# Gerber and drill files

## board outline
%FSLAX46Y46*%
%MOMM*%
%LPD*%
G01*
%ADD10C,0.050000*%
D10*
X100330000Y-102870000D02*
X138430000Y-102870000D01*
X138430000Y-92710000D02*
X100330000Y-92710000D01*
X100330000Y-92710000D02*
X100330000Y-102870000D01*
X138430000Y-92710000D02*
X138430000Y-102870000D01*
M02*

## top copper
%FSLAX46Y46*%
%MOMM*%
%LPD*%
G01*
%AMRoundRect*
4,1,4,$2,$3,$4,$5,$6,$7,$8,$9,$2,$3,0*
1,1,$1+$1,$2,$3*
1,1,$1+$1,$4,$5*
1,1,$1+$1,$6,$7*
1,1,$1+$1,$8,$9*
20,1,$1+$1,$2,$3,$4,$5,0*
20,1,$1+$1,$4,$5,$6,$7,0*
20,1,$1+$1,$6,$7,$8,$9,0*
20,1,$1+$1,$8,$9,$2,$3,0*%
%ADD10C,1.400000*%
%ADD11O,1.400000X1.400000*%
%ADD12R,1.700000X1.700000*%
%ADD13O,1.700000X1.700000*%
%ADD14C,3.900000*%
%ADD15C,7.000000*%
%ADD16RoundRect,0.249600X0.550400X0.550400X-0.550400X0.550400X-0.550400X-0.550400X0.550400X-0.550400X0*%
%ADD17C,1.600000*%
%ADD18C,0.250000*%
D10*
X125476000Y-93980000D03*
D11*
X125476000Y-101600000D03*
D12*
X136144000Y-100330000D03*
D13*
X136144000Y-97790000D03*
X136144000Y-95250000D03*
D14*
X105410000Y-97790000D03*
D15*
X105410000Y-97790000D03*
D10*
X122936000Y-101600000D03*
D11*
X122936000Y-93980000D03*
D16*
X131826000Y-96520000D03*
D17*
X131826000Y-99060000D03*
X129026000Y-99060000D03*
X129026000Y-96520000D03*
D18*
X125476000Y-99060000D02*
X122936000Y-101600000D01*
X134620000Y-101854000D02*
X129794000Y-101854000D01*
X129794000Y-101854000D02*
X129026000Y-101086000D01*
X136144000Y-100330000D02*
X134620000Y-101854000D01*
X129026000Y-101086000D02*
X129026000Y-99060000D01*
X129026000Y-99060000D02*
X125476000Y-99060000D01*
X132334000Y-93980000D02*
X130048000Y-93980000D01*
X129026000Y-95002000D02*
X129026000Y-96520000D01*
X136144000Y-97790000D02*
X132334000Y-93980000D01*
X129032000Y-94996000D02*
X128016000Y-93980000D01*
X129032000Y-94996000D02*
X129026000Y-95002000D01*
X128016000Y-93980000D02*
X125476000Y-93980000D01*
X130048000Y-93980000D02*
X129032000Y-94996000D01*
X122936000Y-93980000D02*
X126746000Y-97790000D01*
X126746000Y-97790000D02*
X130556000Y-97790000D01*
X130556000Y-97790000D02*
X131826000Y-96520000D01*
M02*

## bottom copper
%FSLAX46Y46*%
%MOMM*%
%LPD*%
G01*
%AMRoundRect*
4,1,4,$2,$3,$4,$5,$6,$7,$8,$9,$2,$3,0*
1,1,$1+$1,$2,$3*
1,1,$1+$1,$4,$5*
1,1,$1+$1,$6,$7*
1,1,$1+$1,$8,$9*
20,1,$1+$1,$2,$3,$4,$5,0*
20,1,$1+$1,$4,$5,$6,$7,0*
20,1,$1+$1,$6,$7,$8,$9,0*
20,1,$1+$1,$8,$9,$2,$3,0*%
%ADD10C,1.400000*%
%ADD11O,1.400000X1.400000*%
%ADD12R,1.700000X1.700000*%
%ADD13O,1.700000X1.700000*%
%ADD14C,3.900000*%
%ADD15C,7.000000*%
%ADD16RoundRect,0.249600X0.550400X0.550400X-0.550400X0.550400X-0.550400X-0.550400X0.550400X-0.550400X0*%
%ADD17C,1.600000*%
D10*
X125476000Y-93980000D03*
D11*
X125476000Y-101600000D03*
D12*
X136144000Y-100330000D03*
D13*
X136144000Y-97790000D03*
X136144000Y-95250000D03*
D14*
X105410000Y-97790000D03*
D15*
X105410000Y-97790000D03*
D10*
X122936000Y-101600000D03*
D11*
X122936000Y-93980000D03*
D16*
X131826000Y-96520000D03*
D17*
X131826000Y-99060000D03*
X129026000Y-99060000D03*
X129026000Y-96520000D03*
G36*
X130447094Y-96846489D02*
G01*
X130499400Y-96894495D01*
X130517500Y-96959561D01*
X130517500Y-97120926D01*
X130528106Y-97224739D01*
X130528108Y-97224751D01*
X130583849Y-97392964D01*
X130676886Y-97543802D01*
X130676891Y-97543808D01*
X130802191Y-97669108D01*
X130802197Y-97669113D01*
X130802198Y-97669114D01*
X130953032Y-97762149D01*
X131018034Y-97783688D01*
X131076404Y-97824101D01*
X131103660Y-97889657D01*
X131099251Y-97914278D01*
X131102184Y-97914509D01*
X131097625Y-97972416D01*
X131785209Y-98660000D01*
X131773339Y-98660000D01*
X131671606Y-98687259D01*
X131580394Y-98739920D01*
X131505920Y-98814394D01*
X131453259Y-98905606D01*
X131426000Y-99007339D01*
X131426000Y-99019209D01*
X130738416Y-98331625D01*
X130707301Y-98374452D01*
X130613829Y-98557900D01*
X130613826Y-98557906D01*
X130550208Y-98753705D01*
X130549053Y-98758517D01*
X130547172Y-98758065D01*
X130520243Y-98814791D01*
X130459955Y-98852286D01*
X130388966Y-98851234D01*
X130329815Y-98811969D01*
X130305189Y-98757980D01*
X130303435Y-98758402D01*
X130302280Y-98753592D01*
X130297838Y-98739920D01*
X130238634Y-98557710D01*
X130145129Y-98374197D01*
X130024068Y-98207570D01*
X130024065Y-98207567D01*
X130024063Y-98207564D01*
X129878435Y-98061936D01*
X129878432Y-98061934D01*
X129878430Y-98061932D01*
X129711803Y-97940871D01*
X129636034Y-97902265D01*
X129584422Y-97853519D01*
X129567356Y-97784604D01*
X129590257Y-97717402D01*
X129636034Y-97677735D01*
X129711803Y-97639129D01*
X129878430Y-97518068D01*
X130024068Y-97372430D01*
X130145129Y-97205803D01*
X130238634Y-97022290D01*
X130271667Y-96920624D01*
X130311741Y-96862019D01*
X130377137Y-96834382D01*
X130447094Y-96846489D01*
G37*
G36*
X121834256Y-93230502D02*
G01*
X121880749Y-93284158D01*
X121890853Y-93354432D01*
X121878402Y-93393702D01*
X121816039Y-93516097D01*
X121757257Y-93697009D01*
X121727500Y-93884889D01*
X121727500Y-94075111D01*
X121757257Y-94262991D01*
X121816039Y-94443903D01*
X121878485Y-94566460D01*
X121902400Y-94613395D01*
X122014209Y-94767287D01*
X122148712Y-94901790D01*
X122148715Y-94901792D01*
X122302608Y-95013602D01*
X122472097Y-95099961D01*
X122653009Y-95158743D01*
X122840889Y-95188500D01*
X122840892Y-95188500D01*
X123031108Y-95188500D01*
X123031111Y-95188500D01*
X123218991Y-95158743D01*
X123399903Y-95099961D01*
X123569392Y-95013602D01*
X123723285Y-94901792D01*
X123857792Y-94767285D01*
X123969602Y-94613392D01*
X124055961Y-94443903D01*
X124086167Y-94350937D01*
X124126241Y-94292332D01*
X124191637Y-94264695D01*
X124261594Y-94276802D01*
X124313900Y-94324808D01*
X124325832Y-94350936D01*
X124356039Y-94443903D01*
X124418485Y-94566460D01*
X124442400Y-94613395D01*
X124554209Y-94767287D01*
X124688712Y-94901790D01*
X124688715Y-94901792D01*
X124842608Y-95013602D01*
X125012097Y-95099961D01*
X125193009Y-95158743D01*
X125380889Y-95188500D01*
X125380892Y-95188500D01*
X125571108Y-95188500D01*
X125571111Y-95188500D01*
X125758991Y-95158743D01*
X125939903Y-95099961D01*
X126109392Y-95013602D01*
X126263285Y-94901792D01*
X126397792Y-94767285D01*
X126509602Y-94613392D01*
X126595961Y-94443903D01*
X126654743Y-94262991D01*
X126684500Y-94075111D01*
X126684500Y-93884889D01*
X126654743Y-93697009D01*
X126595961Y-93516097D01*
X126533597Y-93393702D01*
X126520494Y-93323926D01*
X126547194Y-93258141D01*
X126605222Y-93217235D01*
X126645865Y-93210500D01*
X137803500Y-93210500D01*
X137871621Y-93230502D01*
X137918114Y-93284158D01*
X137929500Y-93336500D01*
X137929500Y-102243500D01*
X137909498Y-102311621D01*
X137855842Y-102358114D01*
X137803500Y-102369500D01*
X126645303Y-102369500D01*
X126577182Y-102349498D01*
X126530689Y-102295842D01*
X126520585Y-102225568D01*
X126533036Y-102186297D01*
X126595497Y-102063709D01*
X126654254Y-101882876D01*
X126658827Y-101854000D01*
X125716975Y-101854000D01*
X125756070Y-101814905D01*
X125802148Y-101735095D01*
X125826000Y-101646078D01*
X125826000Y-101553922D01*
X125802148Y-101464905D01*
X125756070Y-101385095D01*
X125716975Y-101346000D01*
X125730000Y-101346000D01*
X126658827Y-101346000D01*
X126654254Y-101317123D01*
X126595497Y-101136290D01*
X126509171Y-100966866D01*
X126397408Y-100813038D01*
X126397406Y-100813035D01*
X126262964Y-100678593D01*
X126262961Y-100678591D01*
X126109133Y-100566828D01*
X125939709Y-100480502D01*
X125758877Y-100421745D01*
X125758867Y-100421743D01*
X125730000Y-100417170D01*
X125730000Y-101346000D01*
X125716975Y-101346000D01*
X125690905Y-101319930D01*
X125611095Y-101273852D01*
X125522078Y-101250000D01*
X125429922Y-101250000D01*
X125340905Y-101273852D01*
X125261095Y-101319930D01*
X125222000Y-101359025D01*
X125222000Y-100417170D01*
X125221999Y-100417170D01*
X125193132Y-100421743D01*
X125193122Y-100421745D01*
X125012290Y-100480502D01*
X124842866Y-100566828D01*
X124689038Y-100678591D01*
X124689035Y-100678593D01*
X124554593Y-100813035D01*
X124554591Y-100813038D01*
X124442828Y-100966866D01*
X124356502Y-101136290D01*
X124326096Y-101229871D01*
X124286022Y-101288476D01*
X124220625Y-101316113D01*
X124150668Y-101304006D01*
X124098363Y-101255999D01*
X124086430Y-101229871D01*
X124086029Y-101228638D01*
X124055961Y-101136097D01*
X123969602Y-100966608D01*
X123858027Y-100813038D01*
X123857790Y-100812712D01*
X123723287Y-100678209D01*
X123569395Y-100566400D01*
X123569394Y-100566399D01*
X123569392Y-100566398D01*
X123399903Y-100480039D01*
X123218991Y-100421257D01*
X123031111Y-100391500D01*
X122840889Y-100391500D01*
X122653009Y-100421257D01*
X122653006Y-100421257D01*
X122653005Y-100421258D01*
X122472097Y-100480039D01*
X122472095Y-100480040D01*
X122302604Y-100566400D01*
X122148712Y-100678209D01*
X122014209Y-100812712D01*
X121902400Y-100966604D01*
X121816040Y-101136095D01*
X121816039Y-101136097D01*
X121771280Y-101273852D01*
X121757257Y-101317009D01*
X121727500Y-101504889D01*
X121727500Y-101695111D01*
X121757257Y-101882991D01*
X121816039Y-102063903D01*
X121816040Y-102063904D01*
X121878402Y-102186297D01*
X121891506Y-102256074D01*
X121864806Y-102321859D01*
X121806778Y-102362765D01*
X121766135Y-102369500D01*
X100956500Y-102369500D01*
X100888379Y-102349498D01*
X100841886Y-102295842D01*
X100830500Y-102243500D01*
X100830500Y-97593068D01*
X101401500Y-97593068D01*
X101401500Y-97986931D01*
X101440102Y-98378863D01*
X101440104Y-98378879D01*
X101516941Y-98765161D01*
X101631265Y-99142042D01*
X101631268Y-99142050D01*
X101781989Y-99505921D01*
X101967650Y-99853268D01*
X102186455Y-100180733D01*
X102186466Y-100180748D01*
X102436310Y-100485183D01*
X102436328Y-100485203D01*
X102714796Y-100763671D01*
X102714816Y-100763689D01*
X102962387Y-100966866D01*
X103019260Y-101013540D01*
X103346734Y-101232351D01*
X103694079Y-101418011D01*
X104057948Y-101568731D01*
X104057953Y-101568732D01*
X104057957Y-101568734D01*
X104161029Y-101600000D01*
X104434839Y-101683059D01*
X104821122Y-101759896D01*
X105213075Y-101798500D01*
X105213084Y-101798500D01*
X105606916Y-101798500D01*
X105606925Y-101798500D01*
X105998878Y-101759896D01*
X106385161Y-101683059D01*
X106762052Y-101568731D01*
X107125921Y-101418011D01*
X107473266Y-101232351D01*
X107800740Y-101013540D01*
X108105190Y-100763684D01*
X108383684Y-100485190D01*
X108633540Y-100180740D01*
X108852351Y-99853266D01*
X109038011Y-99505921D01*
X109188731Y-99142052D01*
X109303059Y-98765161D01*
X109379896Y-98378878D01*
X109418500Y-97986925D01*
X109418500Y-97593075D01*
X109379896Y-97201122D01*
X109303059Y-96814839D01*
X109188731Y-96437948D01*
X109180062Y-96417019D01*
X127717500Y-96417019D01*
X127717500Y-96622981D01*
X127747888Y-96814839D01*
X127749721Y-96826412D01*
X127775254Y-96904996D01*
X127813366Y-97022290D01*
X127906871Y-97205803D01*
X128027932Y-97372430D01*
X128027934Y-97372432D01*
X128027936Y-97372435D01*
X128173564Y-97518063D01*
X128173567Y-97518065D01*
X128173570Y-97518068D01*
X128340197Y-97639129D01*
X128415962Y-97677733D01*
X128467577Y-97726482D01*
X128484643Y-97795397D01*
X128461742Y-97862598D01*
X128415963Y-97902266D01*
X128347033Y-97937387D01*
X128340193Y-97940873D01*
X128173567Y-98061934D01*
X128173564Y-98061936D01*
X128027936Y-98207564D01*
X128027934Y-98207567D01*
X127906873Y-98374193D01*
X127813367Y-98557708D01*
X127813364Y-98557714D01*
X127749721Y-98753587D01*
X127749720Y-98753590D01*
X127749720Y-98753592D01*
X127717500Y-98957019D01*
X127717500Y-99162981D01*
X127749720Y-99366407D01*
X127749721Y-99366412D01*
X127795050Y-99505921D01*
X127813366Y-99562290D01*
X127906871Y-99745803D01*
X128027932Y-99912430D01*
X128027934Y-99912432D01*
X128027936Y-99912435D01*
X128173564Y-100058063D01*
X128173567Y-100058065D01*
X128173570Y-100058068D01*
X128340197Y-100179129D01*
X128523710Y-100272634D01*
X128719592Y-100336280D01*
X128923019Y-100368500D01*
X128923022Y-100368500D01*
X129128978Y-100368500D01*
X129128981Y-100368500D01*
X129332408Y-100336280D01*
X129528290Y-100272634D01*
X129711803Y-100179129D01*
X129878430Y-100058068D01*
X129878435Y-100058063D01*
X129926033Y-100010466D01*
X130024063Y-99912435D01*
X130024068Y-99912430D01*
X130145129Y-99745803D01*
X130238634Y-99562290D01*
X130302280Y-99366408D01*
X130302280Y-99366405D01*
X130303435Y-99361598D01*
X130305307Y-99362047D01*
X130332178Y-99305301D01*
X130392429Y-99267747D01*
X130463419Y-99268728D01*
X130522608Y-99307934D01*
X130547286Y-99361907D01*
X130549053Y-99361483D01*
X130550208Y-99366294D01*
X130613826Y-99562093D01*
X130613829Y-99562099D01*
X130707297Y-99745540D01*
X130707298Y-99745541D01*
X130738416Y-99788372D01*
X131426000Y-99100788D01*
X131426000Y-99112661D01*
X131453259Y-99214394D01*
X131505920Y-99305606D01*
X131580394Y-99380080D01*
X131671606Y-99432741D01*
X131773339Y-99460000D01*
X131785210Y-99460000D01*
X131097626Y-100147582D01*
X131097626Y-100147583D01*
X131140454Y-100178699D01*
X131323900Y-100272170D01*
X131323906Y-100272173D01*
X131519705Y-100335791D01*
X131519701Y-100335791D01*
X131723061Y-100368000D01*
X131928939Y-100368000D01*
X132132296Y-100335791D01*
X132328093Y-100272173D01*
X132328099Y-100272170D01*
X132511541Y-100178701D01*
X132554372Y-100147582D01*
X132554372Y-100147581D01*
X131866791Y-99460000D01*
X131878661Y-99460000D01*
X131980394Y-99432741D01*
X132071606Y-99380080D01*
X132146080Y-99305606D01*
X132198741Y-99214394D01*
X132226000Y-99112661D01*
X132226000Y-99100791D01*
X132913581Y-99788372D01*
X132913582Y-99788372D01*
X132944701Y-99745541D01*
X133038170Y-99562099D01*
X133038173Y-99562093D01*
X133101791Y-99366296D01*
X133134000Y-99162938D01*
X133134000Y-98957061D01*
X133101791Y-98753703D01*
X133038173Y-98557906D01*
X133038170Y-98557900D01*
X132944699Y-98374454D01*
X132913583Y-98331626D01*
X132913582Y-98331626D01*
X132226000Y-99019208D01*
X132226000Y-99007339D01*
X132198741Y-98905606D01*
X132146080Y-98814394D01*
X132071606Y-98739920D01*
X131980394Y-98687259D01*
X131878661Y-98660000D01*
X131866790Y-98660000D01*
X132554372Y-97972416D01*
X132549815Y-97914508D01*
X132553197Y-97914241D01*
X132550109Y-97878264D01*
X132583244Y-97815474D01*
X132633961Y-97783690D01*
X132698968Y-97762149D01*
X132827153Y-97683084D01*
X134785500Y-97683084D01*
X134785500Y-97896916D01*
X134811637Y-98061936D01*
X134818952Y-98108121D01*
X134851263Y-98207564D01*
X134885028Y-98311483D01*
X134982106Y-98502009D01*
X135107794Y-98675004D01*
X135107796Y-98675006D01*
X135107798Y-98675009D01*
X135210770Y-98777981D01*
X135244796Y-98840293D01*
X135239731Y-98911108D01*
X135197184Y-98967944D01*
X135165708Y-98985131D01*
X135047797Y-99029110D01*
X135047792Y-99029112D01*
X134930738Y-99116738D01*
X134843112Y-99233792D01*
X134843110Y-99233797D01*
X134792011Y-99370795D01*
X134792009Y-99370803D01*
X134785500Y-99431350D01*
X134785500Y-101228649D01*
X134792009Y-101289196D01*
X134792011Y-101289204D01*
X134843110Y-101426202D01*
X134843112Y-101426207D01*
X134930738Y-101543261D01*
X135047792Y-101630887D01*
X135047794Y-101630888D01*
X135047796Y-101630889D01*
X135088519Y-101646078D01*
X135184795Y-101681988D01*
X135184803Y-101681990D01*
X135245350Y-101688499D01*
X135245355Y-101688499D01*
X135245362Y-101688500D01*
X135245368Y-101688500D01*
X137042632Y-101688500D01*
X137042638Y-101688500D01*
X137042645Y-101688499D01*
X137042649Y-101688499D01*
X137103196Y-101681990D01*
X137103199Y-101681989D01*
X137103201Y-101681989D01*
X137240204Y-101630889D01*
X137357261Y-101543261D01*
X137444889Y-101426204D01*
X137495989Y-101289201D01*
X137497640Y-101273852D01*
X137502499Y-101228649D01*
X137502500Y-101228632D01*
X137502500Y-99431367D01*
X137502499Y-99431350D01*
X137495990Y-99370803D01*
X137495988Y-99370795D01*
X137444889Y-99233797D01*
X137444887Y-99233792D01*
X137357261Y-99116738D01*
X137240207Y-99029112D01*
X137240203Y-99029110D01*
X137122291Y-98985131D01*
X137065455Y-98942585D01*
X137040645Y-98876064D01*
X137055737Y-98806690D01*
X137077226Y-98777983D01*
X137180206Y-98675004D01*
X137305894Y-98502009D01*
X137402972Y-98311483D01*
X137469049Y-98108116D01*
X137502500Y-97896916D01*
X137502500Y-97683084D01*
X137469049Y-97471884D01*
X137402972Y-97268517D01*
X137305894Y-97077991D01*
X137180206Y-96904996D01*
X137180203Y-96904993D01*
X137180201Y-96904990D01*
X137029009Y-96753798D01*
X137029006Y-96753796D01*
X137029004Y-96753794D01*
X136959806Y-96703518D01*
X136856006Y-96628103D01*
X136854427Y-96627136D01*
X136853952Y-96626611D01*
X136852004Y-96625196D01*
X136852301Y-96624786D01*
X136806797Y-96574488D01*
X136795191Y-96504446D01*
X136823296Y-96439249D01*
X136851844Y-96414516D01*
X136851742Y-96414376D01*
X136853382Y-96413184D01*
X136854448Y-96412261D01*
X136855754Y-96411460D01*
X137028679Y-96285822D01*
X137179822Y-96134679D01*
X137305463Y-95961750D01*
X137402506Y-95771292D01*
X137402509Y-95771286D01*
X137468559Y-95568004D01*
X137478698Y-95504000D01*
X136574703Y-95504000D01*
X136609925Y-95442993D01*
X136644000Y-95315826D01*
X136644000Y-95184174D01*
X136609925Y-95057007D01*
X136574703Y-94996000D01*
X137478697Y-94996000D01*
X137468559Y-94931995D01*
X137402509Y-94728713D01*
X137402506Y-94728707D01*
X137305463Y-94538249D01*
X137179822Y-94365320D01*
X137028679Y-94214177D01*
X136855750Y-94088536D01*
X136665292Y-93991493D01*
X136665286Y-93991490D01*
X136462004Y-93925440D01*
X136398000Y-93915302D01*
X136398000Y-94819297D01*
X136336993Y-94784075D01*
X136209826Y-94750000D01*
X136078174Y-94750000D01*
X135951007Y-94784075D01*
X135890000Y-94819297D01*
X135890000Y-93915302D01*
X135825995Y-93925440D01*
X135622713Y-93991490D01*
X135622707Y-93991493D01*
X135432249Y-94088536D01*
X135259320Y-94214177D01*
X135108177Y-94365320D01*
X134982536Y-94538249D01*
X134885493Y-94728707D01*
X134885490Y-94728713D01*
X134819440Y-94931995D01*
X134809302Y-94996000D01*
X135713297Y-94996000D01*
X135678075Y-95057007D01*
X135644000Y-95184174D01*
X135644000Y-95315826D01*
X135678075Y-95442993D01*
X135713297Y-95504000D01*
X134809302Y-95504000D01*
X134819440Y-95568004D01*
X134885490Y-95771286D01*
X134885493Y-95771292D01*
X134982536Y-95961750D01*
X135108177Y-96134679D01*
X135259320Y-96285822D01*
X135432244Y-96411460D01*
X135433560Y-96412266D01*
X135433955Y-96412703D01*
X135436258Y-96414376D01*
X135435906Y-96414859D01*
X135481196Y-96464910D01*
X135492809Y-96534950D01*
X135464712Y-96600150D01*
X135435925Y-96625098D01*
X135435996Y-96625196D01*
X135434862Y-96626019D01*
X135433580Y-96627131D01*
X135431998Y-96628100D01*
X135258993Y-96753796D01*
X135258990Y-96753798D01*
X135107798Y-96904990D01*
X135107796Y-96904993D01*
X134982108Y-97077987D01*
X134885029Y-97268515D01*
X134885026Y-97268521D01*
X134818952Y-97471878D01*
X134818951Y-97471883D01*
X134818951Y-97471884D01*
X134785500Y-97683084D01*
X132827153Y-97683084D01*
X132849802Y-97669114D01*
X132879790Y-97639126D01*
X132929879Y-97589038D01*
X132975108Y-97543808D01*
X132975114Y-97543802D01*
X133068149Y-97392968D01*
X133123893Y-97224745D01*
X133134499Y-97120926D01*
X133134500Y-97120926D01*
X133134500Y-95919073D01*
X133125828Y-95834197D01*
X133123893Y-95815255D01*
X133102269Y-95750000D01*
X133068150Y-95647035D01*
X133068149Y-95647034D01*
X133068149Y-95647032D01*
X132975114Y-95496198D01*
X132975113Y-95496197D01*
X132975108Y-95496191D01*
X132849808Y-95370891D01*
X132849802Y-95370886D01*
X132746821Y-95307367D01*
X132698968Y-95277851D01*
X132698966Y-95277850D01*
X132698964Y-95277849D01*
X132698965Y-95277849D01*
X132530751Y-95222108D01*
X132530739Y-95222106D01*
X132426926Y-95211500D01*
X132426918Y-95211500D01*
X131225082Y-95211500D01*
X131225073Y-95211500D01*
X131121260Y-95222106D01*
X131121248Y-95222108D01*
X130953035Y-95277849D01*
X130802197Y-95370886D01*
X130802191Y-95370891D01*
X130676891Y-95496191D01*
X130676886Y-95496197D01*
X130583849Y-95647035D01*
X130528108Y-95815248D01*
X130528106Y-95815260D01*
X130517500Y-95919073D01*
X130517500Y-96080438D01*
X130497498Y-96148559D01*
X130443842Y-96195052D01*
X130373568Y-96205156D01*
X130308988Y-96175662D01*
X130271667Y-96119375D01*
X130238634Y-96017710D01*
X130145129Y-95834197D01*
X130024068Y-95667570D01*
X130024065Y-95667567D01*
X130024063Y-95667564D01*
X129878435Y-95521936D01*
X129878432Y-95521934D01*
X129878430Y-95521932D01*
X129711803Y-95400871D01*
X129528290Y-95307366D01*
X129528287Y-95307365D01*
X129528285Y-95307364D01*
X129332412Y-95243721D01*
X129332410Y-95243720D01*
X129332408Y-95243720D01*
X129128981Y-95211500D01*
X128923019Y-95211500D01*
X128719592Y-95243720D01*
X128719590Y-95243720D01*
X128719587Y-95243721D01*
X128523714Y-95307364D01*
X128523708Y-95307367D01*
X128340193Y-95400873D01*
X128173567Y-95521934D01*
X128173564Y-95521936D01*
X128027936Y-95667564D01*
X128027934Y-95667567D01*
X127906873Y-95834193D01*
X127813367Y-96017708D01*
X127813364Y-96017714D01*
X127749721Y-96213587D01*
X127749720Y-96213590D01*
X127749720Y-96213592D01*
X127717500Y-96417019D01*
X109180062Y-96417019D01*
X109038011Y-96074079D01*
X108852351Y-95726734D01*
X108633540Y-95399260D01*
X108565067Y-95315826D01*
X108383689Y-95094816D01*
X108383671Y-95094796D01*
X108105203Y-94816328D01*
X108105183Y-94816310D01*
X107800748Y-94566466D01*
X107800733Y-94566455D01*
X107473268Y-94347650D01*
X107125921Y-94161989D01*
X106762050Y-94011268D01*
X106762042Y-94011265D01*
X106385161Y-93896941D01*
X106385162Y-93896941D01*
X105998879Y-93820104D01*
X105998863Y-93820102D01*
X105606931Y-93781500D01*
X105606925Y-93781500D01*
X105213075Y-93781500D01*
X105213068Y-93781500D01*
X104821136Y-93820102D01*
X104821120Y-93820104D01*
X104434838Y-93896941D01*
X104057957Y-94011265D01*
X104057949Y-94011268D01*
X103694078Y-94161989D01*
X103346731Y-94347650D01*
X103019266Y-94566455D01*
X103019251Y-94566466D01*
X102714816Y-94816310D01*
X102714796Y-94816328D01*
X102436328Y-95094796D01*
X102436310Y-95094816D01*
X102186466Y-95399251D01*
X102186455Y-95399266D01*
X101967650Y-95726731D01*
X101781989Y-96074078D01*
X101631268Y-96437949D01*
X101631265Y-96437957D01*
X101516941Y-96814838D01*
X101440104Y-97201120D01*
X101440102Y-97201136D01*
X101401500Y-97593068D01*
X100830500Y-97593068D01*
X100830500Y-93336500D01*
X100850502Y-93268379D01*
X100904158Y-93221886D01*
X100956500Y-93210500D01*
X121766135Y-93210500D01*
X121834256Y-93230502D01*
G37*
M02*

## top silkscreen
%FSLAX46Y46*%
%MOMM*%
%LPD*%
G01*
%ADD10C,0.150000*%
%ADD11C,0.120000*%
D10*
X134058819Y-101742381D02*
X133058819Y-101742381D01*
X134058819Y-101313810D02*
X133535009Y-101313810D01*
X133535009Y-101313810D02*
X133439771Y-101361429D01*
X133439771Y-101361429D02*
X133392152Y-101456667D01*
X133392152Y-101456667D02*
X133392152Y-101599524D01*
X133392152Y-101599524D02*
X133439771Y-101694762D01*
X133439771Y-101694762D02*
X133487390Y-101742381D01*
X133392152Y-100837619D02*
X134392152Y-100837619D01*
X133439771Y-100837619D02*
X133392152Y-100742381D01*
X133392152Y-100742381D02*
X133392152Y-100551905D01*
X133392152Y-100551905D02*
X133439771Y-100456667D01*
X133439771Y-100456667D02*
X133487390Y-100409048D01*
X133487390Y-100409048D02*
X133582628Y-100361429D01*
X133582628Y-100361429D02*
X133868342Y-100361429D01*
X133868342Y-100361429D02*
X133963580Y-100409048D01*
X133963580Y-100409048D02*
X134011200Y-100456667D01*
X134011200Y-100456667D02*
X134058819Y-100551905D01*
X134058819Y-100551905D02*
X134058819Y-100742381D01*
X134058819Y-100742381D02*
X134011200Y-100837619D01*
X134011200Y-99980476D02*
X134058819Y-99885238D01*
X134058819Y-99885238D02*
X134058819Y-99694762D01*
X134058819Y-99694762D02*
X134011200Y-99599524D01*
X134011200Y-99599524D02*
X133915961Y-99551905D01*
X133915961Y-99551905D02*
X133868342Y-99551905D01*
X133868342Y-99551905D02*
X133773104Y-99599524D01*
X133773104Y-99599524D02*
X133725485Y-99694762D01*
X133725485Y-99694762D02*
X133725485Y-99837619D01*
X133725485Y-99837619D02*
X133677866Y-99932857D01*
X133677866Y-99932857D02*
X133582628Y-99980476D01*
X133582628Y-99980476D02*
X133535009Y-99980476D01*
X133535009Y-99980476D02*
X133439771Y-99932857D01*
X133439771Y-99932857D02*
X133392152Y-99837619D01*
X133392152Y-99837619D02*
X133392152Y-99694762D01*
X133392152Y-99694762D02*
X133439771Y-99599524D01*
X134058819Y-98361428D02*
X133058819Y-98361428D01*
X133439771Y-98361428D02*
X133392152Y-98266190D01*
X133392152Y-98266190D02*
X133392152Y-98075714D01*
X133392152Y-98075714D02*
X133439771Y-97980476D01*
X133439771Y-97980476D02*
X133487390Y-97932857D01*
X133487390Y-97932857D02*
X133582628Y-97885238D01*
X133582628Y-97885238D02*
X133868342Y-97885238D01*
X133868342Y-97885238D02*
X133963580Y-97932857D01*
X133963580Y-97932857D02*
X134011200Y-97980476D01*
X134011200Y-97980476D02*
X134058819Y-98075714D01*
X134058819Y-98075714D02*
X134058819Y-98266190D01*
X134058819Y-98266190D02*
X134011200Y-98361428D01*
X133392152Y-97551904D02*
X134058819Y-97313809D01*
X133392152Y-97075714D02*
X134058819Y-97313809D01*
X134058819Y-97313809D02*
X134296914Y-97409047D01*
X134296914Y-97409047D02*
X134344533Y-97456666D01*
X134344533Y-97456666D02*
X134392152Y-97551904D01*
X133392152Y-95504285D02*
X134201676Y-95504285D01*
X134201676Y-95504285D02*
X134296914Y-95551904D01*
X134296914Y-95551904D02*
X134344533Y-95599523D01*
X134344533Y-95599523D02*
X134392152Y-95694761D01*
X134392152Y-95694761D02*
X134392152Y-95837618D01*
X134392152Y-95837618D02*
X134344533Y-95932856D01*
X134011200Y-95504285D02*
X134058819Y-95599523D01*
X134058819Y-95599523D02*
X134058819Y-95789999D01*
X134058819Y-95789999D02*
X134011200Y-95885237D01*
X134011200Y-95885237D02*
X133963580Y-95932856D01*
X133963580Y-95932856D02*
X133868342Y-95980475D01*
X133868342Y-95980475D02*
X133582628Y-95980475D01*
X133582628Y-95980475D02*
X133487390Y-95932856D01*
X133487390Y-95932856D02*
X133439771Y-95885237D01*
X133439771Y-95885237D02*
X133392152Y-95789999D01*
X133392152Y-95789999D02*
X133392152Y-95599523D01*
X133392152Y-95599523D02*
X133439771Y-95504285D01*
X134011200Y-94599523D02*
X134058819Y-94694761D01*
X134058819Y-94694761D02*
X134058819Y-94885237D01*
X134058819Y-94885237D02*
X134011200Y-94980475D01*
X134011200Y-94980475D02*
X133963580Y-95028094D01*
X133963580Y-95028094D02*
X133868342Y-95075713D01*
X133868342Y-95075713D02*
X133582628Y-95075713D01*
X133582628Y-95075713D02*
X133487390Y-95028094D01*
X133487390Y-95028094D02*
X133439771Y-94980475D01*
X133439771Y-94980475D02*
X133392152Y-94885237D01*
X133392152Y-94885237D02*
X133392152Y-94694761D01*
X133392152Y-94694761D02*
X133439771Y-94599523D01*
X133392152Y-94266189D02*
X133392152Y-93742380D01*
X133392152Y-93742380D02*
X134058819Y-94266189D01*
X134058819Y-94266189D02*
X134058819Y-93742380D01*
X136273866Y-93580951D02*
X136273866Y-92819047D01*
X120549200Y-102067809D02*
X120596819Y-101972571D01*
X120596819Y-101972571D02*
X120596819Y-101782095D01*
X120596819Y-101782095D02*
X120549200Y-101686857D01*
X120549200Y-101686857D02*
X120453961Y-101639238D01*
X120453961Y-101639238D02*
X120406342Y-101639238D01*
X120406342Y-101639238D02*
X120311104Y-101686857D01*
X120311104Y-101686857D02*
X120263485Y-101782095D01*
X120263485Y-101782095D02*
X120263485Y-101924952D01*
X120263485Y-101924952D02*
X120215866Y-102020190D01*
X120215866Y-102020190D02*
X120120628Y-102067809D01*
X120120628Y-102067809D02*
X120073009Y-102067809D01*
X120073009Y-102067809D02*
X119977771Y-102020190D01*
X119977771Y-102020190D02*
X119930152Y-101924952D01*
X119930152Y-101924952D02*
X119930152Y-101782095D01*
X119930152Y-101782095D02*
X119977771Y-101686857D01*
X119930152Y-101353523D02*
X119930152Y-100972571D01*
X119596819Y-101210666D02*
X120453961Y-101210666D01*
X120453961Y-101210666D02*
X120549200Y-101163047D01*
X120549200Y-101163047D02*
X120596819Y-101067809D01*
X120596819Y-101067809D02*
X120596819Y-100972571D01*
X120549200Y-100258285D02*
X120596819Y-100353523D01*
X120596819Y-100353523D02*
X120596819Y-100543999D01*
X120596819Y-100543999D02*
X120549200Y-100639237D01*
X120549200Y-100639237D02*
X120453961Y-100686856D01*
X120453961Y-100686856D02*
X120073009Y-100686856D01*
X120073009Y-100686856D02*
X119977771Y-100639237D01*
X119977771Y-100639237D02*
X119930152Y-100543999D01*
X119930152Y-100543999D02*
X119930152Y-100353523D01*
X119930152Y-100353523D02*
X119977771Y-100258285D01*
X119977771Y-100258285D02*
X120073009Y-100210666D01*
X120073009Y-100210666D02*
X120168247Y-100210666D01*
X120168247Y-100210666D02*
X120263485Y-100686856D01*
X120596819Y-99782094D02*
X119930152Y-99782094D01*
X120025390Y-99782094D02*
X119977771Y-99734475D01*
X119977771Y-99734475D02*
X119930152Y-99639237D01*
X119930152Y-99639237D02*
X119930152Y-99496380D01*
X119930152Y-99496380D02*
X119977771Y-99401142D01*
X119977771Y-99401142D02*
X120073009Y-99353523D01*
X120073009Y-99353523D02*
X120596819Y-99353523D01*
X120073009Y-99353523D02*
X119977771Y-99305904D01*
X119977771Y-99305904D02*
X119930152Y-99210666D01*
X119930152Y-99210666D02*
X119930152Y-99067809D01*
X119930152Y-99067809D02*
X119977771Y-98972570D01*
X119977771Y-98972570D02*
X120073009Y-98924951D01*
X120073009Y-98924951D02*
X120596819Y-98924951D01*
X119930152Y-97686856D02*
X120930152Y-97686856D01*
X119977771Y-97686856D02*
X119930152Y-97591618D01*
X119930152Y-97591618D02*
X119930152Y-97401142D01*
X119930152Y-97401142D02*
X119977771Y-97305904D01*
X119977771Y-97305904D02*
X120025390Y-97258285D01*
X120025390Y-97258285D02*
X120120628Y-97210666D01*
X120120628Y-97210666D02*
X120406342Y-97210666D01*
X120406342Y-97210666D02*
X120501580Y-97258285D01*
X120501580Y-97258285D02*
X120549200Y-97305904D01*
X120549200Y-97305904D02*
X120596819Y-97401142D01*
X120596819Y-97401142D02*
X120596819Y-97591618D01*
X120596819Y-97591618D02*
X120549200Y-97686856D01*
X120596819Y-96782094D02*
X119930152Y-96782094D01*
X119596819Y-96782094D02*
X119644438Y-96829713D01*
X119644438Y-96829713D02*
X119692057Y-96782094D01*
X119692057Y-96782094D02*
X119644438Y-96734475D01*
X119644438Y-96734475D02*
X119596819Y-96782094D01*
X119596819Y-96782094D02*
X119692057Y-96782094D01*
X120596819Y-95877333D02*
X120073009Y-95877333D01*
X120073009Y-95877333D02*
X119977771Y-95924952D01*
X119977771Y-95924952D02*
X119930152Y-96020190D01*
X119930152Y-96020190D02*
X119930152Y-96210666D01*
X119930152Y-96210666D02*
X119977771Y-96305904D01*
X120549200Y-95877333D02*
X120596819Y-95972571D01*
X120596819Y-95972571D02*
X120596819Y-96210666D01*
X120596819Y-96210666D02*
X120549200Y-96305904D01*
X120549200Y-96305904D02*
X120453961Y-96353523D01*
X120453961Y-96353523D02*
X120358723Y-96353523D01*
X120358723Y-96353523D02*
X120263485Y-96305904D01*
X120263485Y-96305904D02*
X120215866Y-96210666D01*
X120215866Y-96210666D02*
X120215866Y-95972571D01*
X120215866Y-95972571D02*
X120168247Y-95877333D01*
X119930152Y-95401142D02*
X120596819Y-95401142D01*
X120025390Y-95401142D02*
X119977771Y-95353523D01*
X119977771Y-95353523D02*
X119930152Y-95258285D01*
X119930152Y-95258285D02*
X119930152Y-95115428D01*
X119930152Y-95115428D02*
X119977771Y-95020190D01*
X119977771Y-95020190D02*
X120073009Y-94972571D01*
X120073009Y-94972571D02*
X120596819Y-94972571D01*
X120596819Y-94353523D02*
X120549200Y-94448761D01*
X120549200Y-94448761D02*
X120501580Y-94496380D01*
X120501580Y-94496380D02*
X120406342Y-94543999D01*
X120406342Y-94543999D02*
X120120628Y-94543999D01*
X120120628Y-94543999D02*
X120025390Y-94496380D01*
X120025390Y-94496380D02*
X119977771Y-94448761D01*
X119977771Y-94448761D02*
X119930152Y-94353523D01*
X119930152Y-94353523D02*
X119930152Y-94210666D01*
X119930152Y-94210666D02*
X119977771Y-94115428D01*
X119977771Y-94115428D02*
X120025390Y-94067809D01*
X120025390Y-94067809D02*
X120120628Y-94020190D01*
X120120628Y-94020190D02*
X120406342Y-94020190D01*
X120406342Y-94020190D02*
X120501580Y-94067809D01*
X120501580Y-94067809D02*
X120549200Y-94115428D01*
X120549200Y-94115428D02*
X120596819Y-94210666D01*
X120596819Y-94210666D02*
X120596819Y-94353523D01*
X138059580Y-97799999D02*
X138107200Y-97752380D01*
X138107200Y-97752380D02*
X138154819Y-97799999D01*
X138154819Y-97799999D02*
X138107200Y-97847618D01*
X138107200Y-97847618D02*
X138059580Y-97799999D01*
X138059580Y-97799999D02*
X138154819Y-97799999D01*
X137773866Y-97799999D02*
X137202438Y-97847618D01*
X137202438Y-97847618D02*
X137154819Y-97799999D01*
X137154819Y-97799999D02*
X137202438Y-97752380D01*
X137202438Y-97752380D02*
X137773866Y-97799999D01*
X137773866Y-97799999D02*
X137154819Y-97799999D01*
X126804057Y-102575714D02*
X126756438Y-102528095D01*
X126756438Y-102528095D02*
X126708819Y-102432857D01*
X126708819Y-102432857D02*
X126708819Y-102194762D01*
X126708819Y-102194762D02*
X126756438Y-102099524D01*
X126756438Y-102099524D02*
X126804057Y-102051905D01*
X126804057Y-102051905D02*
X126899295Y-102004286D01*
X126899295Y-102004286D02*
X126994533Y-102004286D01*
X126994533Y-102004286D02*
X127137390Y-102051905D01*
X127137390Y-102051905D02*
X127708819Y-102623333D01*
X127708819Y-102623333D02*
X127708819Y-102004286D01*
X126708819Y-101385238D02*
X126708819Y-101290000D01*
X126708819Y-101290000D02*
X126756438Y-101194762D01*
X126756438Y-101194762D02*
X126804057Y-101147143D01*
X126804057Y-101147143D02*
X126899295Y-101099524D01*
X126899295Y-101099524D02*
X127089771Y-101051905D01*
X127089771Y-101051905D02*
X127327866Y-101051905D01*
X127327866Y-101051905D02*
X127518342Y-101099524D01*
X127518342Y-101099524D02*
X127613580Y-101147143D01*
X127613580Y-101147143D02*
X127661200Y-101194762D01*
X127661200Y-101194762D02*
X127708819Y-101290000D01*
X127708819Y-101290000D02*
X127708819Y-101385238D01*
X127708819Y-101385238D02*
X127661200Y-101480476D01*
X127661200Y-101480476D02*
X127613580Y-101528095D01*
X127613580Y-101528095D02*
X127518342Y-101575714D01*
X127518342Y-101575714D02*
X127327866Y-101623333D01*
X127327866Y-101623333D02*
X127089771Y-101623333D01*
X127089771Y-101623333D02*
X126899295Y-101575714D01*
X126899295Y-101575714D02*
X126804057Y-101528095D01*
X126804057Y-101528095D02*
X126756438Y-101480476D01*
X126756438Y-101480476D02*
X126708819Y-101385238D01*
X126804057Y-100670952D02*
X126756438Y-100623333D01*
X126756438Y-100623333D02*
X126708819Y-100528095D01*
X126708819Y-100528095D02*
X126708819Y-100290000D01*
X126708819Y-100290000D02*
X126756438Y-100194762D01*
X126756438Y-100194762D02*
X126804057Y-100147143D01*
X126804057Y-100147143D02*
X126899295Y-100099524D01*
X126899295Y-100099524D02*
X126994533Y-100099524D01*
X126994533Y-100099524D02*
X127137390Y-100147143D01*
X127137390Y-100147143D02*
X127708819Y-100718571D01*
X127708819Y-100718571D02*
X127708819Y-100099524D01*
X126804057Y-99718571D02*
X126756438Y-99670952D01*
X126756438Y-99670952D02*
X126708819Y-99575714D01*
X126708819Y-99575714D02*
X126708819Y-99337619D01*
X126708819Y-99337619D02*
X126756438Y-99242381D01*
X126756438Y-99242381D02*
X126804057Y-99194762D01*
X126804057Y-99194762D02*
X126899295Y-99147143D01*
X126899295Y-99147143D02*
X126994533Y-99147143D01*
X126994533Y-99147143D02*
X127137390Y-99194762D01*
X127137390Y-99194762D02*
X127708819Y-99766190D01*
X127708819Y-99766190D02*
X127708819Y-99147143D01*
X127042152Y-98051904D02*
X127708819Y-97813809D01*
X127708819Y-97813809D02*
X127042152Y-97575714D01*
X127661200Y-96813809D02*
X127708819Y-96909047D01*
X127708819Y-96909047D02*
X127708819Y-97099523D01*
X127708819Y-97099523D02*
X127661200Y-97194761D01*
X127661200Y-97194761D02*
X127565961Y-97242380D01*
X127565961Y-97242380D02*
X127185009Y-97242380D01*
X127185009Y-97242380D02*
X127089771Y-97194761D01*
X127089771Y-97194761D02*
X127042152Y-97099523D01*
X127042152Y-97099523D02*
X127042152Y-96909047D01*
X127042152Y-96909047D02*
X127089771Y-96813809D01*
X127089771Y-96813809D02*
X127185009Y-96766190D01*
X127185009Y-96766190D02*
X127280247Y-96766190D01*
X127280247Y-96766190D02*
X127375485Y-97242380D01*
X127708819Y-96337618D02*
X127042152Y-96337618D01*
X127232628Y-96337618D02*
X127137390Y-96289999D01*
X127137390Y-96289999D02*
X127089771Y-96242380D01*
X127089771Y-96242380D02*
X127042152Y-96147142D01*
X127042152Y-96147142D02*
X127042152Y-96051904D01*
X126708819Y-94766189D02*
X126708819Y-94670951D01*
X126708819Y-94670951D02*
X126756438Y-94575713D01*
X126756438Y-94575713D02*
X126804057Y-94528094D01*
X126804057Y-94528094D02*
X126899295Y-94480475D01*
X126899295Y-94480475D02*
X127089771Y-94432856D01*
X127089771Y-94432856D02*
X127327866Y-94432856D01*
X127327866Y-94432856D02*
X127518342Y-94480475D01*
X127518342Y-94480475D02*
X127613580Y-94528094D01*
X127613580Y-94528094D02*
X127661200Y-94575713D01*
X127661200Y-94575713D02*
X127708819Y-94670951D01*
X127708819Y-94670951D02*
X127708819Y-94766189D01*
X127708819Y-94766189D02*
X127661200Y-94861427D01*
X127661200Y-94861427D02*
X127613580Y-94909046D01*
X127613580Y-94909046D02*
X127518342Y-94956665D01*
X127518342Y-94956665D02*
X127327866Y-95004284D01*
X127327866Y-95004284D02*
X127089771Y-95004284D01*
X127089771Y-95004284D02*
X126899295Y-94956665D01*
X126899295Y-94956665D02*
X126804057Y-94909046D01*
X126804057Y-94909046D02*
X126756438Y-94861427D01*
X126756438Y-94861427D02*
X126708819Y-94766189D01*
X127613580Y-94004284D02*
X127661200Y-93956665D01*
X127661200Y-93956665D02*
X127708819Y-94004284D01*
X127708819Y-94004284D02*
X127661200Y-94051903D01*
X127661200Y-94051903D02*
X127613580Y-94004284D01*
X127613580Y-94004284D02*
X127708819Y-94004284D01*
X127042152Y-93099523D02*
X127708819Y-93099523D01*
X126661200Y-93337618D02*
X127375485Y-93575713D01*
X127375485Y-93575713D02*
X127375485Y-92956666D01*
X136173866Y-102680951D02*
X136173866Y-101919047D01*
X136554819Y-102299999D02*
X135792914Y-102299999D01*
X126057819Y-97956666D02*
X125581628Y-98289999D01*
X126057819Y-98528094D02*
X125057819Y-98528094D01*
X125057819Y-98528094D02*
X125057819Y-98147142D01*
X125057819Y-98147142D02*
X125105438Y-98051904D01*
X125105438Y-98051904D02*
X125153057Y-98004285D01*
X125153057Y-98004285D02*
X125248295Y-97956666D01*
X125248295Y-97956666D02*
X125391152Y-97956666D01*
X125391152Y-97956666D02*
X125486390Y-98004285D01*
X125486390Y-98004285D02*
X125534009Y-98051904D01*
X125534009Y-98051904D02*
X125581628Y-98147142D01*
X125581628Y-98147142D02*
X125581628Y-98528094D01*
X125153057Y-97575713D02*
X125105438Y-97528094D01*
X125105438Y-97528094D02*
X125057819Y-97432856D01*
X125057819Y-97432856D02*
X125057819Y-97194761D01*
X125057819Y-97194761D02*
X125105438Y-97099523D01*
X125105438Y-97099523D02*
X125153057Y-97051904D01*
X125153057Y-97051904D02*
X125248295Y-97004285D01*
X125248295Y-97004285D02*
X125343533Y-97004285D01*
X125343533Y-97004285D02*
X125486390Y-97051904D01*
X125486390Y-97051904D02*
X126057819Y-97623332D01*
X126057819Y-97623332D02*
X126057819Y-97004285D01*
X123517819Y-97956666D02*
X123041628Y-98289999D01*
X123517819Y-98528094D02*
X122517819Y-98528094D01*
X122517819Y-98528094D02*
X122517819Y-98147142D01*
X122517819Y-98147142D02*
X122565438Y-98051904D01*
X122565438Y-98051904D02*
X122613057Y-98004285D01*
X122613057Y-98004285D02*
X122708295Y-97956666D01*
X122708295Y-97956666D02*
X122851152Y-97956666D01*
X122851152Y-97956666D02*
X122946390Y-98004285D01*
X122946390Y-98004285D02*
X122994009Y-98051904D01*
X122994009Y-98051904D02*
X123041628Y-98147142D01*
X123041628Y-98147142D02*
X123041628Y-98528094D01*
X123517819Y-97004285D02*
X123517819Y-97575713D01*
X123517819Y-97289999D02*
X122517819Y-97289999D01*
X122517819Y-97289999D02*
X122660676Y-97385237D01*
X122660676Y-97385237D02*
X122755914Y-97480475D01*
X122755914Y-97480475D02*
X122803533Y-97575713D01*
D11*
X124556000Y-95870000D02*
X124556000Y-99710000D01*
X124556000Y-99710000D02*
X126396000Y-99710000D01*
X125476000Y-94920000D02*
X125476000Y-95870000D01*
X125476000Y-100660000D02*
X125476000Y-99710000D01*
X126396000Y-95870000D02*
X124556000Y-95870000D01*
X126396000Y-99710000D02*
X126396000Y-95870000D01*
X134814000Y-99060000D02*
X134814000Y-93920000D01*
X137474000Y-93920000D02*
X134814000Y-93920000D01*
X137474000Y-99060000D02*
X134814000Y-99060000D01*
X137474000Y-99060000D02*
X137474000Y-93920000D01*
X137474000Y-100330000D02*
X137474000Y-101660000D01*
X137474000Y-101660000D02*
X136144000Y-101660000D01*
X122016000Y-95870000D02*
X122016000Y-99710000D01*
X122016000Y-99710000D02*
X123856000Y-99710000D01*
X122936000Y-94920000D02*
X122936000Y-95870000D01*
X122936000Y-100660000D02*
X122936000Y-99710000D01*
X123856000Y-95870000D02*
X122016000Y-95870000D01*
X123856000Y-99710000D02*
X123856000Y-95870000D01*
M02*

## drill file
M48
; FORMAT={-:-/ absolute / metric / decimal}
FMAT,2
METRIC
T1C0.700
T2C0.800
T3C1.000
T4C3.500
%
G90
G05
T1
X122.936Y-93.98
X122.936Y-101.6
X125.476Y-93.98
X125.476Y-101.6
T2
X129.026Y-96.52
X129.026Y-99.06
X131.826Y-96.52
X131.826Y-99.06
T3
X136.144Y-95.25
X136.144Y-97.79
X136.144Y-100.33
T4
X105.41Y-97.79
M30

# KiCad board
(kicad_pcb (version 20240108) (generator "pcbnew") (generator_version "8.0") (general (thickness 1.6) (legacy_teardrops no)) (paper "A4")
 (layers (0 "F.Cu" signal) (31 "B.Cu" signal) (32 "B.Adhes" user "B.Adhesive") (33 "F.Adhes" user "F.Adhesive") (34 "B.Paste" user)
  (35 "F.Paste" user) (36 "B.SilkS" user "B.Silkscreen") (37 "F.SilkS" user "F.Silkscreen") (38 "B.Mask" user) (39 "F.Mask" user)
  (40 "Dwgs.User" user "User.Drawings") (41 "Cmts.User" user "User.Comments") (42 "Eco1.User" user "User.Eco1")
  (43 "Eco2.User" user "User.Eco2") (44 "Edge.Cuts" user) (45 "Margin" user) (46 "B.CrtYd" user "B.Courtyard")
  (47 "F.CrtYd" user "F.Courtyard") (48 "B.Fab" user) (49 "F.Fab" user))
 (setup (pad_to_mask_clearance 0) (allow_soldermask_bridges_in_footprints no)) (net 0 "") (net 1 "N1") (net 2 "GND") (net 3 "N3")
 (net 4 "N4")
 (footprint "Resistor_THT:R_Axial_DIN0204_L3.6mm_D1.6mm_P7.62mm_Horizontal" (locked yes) (layer "F.Cu") (at 125.476 93.98 -90)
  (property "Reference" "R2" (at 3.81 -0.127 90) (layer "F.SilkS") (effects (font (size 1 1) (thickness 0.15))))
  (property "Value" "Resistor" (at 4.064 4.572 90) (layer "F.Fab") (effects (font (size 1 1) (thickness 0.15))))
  (fp_line (start 1.89 0.92) (end 5.73 0.92) (stroke (width 0.12) (type solid)) (layer "F.SilkS"))
  (fp_line (start 5.73 0.92) (end 5.73 -0.92) (stroke (width 0.12) (type solid)) (layer "F.SilkS"))
  (fp_line (start 0.94 0) (end 1.89 0) (stroke (width 0.12) (type solid)) (layer "F.SilkS"))
  (fp_line (start 6.68 0) (end 5.73 0) (stroke (width 0.12) (type solid)) (layer "F.SilkS"))
  (fp_line (start 1.89 -0.92) (end 1.89 0.92) (stroke (width 0.12) (type solid)) (layer "F.SilkS"))
  (fp_line (start 5.73 -0.92) (end 1.89 -0.92) (stroke (width 0.12) (type solid)) (layer "F.SilkS"))
  (pad "1" thru_hole circle (at 0 0 270) (size 1.4 1.4) (drill 0.7) (layers "*.Cu" "*.Mask") (remove_unused_layers no) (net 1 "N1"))
  (pad "2" thru_hole oval (at 7.62 0 270) (size 1.4 1.4) (drill 0.7) (layers "*.Cu" "*.Mask") (remove_unused_layers no) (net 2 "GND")))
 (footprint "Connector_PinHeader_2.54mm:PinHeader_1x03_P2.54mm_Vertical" (layer "F.Cu") (at 136.144 100.33 180)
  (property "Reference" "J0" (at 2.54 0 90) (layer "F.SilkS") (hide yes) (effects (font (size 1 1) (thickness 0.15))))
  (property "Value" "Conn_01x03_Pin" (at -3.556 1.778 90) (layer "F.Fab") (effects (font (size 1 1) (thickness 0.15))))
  (fp_line (start 1.33 1.27) (end 1.33 6.41) (stroke (width 0.12) (type solid)) (layer "F.SilkS"))
  (fp_line (start -1.33 6.41) (end 1.33 6.41) (stroke (width 0.12) (type solid)) (layer "F.SilkS"))
  (fp_line (start -1.33 1.27) (end 1.33 1.27) (stroke (width 0.12) (type solid)) (layer "F.SilkS"))
  (fp_line (start -1.33 1.27) (end -1.33 6.41) (stroke (width 0.12) (type solid)) (layer "F.SilkS"))
  (fp_line (start -1.33 0) (end -1.33 -1.33) (stroke (width 0.12) (type solid)) (layer "F.SilkS"))
  (fp_line (start -1.33 -1.33) (end 0 -1.33) (stroke (width 0.12) (type solid)) (layer "F.SilkS"))
  (pad "1" thru_hole rect (at 0 0 180) (size 1.7 1.7) (drill 1) (layers "*.Cu" "*.Mask") (remove_unused_layers no) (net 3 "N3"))
  (pad "2" thru_hole oval (at 0 2.54 180) (size 1.7 1.7) (drill 1) (layers "*.Cu" "*.Mask") (remove_unused_layers no) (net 1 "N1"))
  (pad "3" thru_hole oval (at 0 5.08 180) (size 1.7 1.7) (drill 1) (layers "*.Cu" "*.Mask") (remove_unused_layers no) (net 2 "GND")))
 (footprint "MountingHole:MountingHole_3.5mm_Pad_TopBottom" (layer "F.Cu") (at 105.41 97.79)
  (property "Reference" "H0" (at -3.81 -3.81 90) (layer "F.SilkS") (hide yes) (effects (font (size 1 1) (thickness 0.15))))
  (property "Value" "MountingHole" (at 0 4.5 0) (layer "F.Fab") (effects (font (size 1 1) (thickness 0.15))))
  (pad "1" thru_hole circle (at 0 0) (size 3.9 3.9) (drill 3.5) (layers "*.Cu" "*.Mask") (remove_unused_layers no))
  (pad "1" connect circle (at 0 0) (size 7 7) (layers "F.Cu" "F.Mask"))
  (pad "1" connect circle (at 0 0) (size 7 7) (layers "B.Cu" "B.Mask")))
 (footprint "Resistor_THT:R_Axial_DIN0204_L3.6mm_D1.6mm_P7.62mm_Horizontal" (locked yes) (layer "F.Cu") (at 122.936 101.6 90)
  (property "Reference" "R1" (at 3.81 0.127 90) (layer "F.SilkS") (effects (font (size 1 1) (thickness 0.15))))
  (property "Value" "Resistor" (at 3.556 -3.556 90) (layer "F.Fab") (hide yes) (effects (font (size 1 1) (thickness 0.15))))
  (fp_line (start 5.73 -0.92) (end 1.89 -0.92) (stroke (width 0.12) (type solid)) (layer "F.SilkS"))
  (fp_line (start 1.89 -0.92) (end 1.89 0.92) (stroke (width 0.12) (type solid)) (layer "F.SilkS"))
  (fp_line (start 6.68 0) (end 5.73 0) (stroke (width 0.12) (type solid)) (layer "F.SilkS"))
  (fp_line (start 0.94 0) (end 1.89 0) (stroke (width 0.12) (type solid)) (layer "F.SilkS"))
  (fp_line (start 5.73 0.92) (end 5.73 -0.92) (stroke (width 0.12) (type solid)) (layer "F.SilkS"))
  (fp_line (start 1.89 0.92) (end 5.73 0.92) (stroke (width 0.12) (type solid)) (layer "F.SilkS"))
  (pad "1" thru_hole circle (at 0 0 90) (size 1.4 1.4) (drill 0.7) (layers "*.Cu" "*.Mask") (remove_unused_layers no) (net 3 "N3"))
  (pad "2" thru_hole oval (at 7.62 0 90) (size 1.4 1.4) (drill 0.7) (layers "*.Cu" "*.Mask") (remove_unused_layers no) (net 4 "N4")))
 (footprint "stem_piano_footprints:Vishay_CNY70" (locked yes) (layer "B.Cu") (at 131.826 96.52 180)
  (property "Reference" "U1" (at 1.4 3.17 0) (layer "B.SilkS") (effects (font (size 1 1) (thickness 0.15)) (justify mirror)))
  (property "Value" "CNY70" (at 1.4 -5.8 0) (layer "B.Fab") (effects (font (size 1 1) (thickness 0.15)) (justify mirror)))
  (pad "1" thru_hole roundrect (at 0 0 180) (size 1.6 1.6) (drill 0.8) (layers "*.Cu" "*.Mask") (remove_unused_layers no)
   (roundrect_rratio 0.156) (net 4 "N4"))
  (pad "2" thru_hole circle (at 0 -2.54 180) (size 1.6 1.6) (drill 0.8) (layers "*.Cu" "*.Mask") (remove_unused_layers no) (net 2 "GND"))
  (pad "3" thru_hole circle (at 2.8 -2.54 180) (size 1.6 1.6) (drill 0.8) (layers "*.Cu" "*.Mask") (remove_unused_layers no) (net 3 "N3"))
  (pad "4" thru_hole circle (at 2.8 0 180) (size 1.6 1.6) (drill 0.8) (layers "*.Cu" "*.Mask") (remove_unused_layers no) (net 1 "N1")))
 (gr_line (start 100.33 102.87) (end 138.43 102.87) (stroke (width 0.05) (type solid)) (layer "Edge.Cuts"))
 (gr_line (start 138.43 92.71) (end 100.33 92.71) (stroke (width 0.05) (type solid)) (layer "Edge.Cuts"))
 (gr_line (start 100.33 92.71) (end 100.33 102.87) (stroke (width 0.05) (type solid)) (layer "Edge.Cuts"))
 (gr_line (start 138.43 92.71) (end 138.43 102.87) (stroke (width 0.05) (type solid)) (layer "Edge.Cuts"))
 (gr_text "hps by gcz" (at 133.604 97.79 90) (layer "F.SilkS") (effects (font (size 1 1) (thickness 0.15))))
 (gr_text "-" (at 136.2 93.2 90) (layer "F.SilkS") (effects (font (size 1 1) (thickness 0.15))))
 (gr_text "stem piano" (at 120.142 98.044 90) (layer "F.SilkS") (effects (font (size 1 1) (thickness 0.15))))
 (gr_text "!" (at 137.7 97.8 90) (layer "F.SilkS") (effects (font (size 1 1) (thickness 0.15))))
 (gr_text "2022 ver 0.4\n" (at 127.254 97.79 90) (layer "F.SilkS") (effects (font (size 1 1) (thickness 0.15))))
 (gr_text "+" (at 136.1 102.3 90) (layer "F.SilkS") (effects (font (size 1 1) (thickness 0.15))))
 (segment (start 125.476 99.06) (end 122.936 101.6) (width 0.25) (layer "F.Cu") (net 3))
 (segment (start 134.62 101.854) (end 129.794 101.854) (width 0.25) (layer "F.Cu") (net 3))
 (segment (start 129.794 101.854) (end 129.026 101.086) (width 0.25) (layer "F.Cu") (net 3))
 (segment (start 136.144 100.33) (end 134.62 101.854) (width 0.25) (layer "F.Cu") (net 3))
 (segment (start 129.026 101.086) (end 129.026 99.06) (width 0.25) (layer "F.Cu") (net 3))
 (segment (start 129.026 99.06) (end 125.476 99.06) (width 0.25) (layer "F.Cu") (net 3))
 (segment (start 132.334 93.98) (end 130.048 93.98) (width 0.25) (layer "F.Cu") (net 1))
 (segment (start 129.026 95.002) (end 129.026 96.52) (width 0.25) (layer "F.Cu") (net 1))
 (segment (start 136.144 97.79) (end 132.334 93.98) (width 0.25) (layer "F.Cu") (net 1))
 (segment (start 129.032 94.996) (end 128.016 93.98) (width 0.25) (layer "F.Cu") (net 1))
 (segment (start 129.032 94.996) (end 129.026 95.002) (width 0.25) (layer "F.Cu") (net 1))
 (segment (start 128.016 93.98) (end 125.476 93.98) (width 0.25) (layer "F.Cu") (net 1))
 (segment (start 130.048 93.98) (end 129.032 94.996) (width 0.25) (layer "F.Cu") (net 1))
 (segment (start 122.936 93.98) (end 126.746 97.79) (width 0.25) (layer "F.Cu") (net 4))
 (segment (start 126.746 97.79) (end 130.556 97.79) (width 0.25) (layer "F.Cu") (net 4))
 (segment (start 130.556 97.79) (end 131.826 96.52) (width 0.25) (layer "F.Cu") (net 4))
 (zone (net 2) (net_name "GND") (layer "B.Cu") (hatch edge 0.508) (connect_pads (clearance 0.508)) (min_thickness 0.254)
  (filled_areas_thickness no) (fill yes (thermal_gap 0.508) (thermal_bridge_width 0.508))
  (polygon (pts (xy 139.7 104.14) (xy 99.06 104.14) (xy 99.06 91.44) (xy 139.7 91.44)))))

